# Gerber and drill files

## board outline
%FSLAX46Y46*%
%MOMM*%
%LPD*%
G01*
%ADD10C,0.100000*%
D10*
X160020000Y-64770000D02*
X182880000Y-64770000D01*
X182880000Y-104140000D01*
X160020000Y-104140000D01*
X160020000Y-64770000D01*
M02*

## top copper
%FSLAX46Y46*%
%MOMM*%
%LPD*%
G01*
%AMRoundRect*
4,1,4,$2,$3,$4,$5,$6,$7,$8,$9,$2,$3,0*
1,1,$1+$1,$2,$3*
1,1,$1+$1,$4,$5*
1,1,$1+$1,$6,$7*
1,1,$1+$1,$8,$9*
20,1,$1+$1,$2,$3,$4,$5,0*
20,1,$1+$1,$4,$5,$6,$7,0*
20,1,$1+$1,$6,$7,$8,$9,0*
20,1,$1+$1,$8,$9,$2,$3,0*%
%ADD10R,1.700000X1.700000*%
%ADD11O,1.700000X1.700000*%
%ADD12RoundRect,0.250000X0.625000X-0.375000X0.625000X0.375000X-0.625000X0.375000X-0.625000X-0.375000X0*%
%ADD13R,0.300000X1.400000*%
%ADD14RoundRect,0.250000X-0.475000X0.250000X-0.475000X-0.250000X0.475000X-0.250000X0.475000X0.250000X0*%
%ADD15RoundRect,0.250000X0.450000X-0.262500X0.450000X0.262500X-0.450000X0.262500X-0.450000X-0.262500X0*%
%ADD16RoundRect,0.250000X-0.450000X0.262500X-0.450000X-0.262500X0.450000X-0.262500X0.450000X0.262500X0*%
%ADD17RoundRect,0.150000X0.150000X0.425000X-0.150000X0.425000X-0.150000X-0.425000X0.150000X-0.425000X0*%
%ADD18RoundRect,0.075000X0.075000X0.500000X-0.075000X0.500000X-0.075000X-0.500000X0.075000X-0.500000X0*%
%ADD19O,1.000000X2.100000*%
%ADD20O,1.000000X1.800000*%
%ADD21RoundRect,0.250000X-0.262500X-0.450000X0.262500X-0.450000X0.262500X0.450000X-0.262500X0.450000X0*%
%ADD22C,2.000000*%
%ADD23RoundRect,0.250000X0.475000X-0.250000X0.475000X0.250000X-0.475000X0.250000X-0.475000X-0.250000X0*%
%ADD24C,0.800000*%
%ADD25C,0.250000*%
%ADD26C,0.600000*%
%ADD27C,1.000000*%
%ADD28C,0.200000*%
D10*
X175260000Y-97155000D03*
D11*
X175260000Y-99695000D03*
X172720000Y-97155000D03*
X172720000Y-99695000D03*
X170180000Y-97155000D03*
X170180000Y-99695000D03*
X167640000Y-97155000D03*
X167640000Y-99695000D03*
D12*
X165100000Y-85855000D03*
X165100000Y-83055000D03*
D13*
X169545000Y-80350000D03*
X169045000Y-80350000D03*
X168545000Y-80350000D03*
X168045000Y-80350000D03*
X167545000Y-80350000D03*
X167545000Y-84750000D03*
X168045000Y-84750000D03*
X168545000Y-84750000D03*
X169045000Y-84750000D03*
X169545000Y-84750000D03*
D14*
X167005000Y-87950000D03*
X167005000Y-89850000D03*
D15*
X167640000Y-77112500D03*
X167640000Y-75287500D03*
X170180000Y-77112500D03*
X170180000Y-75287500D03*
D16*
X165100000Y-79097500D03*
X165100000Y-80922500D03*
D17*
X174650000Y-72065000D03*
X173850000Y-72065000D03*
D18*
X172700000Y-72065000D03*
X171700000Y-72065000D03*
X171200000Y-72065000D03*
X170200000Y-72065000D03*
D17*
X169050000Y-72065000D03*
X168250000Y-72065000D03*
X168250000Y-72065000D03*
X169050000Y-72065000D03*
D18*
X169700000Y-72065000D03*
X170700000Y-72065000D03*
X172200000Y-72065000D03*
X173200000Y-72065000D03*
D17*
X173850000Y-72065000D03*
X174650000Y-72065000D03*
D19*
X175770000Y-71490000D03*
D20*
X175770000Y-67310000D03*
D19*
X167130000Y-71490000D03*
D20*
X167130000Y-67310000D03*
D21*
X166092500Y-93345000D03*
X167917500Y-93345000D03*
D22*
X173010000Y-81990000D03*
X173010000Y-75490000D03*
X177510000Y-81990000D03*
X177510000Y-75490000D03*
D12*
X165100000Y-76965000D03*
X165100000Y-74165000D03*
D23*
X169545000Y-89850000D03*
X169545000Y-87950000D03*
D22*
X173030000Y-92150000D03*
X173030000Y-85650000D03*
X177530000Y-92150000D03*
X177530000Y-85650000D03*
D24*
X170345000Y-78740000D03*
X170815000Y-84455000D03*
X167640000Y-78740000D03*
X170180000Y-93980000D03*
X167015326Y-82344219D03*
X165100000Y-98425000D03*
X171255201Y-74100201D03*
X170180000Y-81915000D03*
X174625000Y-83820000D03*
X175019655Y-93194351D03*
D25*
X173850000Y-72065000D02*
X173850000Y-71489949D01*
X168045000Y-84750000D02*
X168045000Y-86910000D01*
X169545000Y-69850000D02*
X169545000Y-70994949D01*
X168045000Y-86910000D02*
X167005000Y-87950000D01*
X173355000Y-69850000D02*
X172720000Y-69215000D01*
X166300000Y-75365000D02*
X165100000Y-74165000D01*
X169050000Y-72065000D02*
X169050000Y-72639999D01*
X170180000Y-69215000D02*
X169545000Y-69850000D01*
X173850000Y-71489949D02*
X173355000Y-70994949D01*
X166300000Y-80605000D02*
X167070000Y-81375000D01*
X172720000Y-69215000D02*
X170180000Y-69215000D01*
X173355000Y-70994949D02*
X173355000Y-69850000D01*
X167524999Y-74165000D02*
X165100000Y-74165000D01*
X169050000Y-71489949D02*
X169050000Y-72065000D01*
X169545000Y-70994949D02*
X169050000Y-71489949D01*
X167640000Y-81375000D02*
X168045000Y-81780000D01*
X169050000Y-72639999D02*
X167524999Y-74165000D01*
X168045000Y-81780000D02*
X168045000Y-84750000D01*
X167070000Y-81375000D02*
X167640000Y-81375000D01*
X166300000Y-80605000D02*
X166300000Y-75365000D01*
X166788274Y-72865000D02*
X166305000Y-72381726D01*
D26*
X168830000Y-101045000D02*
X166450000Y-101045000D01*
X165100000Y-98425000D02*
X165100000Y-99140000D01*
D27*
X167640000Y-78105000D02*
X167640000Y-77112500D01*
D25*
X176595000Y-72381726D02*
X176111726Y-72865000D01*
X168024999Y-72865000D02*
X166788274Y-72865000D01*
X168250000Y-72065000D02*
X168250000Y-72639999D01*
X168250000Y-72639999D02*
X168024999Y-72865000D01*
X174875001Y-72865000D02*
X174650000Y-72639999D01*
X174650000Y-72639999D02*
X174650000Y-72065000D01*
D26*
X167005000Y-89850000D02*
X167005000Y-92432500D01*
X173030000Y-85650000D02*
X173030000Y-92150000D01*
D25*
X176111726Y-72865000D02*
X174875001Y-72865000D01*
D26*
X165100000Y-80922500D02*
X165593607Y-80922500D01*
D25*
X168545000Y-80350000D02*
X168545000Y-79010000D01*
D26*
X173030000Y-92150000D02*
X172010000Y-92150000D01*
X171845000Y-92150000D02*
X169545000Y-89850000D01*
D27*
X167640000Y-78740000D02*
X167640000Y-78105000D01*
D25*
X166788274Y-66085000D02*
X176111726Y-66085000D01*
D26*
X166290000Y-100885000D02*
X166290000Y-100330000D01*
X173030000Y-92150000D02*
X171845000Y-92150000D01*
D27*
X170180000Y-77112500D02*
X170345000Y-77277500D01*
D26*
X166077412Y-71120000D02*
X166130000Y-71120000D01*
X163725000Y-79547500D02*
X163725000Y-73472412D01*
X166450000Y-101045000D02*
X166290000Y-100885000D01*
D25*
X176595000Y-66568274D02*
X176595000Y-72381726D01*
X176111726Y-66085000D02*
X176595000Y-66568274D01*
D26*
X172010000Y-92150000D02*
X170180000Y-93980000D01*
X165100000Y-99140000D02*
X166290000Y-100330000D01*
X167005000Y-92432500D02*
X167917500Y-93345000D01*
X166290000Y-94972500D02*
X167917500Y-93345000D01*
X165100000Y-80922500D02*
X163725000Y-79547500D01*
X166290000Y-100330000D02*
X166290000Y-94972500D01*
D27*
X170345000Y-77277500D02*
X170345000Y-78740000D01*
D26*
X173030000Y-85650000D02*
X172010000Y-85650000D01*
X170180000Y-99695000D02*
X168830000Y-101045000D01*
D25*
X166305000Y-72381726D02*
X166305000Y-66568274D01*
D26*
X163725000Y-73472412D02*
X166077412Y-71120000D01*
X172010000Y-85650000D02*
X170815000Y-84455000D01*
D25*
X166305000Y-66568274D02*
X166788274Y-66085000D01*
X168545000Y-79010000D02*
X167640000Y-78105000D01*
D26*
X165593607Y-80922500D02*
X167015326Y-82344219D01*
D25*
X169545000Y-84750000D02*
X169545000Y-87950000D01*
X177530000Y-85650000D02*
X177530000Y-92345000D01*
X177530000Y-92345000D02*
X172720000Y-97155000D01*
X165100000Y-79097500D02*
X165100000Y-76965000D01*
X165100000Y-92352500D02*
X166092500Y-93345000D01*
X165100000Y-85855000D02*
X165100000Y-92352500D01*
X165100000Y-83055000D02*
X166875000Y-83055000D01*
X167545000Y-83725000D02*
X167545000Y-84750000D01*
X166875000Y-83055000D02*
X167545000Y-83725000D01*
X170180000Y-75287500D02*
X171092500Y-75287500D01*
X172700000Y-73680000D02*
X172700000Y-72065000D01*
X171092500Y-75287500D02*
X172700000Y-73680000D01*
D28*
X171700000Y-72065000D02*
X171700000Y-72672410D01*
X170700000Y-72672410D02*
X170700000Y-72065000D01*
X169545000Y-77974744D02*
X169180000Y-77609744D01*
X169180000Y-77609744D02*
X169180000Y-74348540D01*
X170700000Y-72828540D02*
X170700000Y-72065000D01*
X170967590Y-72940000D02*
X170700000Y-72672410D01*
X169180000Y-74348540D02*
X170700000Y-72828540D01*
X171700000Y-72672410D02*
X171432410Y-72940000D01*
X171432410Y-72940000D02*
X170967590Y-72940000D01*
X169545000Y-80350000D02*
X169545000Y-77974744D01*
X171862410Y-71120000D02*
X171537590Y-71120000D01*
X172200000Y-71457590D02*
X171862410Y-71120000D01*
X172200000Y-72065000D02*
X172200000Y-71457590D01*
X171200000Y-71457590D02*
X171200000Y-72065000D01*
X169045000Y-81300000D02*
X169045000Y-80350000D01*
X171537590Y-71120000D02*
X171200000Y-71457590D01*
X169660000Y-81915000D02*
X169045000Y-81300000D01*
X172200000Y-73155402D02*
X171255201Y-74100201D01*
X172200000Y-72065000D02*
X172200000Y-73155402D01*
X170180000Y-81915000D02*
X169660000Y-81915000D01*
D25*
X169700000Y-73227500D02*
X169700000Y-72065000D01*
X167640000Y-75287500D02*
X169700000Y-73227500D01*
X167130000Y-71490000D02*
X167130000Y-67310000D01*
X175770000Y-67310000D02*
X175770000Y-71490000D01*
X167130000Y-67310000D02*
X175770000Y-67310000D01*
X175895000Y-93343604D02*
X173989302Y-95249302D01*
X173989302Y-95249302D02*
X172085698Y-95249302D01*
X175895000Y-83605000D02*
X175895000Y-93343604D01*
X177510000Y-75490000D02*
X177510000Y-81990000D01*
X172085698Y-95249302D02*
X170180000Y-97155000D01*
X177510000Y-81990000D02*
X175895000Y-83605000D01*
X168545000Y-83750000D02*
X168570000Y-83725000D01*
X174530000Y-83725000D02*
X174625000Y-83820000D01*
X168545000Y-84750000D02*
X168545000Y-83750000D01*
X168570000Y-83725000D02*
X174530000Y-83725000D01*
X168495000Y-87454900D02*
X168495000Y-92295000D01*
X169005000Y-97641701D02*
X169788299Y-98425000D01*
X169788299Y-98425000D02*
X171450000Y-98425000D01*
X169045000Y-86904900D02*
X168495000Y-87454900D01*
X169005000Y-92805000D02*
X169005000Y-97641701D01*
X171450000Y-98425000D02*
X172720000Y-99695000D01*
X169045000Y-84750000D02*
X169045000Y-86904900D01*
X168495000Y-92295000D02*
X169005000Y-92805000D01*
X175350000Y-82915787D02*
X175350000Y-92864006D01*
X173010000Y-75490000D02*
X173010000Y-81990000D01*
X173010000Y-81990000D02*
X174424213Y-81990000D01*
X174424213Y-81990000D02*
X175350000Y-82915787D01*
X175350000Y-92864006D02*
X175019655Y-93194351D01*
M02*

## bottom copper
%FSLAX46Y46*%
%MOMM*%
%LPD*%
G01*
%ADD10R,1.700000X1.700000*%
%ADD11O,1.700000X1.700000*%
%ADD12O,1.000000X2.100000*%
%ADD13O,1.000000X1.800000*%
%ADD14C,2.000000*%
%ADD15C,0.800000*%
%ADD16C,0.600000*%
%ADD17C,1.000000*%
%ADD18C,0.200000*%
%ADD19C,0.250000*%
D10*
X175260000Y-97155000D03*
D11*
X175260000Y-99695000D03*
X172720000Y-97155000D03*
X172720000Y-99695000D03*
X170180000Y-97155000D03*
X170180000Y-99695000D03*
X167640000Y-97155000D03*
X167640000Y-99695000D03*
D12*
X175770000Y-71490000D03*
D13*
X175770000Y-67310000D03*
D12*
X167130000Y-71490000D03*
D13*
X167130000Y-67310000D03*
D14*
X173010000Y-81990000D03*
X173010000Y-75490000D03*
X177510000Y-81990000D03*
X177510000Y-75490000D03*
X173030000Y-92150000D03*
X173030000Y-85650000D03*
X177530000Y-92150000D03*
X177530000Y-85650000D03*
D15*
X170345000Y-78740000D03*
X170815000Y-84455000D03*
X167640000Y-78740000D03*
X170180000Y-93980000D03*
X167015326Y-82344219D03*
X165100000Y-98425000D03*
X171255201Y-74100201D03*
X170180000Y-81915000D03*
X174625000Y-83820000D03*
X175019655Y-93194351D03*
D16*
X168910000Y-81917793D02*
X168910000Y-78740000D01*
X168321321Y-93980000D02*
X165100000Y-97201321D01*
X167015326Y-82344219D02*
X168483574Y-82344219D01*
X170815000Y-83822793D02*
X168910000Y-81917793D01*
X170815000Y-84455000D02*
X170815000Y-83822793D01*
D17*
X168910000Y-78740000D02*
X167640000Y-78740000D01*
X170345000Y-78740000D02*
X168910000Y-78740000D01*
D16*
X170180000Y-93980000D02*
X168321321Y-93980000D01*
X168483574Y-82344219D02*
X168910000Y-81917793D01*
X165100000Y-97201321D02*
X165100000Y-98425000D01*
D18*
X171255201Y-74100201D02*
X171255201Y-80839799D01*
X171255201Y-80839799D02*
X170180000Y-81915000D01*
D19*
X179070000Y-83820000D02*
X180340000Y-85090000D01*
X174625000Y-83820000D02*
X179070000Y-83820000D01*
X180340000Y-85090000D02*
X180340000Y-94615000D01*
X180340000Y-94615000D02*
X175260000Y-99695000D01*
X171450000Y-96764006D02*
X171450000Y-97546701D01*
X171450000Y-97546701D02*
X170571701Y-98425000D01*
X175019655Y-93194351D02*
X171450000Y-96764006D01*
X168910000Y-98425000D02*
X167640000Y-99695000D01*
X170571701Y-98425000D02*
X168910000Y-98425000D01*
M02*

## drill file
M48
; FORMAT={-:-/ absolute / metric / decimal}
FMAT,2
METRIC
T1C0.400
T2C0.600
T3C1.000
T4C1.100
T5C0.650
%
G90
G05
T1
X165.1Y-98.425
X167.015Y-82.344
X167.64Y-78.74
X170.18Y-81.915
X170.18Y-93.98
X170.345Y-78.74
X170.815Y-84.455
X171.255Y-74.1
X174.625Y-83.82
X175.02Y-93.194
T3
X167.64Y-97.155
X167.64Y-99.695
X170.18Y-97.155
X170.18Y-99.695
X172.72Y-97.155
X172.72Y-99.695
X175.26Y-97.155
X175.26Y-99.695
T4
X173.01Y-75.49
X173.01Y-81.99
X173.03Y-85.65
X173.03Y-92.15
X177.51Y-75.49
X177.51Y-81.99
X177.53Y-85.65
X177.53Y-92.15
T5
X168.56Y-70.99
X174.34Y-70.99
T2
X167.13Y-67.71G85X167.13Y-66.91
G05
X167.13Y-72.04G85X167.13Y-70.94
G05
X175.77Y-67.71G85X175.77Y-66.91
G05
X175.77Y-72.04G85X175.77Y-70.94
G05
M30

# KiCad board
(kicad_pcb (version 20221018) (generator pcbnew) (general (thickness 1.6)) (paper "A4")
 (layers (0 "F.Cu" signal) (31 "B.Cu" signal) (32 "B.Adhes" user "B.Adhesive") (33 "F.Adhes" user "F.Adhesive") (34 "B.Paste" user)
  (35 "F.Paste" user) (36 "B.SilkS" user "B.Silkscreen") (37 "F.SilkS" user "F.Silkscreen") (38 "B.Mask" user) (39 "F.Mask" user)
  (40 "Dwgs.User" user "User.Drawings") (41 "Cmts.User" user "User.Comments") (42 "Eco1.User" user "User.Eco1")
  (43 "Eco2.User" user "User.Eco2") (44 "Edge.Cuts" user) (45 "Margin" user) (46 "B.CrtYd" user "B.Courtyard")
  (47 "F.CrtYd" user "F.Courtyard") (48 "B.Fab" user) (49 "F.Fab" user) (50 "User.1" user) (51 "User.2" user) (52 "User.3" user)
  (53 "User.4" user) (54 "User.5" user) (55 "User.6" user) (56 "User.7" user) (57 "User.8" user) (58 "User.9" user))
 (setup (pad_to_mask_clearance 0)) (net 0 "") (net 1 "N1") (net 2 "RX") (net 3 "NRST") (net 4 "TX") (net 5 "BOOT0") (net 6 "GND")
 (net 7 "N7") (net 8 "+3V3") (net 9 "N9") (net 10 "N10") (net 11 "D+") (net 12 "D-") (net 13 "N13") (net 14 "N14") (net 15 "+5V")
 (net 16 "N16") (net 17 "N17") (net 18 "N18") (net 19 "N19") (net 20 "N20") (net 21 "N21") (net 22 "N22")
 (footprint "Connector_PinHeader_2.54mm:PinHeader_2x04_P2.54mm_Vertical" (layer "F.Cu") (at 175.26 97.155 -90)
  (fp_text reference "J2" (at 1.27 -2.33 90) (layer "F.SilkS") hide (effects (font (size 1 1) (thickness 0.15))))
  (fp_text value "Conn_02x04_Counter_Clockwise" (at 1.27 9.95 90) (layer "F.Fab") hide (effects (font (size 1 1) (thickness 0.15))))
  (pad "1" thru_hole rect (at 0 0 270) (size 1.7 1.7) (drill 1) (layers "*.Cu" "*.Mask") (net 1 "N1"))
  (pad "2" thru_hole oval (at 2.54 0 270) (size 1.7 1.7) (drill 1) (layers "*.Cu" "*.Mask") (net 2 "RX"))
  (pad "3" thru_hole oval (at 0 2.54 270) (size 1.7 1.7) (drill 1) (layers "*.Cu" "*.Mask") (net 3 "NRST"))
  (pad "4" thru_hole oval (at 2.54 2.54 270) (size 1.7 1.7) (drill 1) (layers "*.Cu" "*.Mask") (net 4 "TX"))
  (pad "5" thru_hole oval (at 0 5.08 270) (size 1.7 1.7) (drill 1) (layers "*.Cu" "*.Mask") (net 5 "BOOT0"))
  (pad "6" thru_hole oval (at 2.54 5.08 270) (size 1.7 1.7) (drill 1) (layers "*.Cu" "*.Mask") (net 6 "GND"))
  (pad "7" thru_hole oval (at 0 7.62 270) (size 1.7 1.7) (drill 1) (layers "*.Cu" "*.Mask") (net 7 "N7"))
  (pad "8" thru_hole oval (at 2.54 7.62 270) (size 1.7 1.7) (drill 1) (layers "*.Cu" "*.Mask") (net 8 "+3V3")))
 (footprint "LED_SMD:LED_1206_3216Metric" (layer "F.Cu") (at 165.1 84.455 90)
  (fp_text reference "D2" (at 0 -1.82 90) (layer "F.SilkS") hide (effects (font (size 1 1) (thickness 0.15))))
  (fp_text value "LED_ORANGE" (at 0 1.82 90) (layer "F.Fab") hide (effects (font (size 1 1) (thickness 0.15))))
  (pad "1" smd roundrect (at -1.4 0 90) (size 1.25 1.75) (layers "F.Cu" "F.Paste" "F.Mask") (roundrect_rratio 0.2) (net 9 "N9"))
  (pad "2" smd roundrect (at 1.4 0 90) (size 1.25 1.75) (layers "F.Cu" "F.Paste" "F.Mask") (roundrect_rratio 0.2) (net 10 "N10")))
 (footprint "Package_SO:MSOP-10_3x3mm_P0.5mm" (layer "F.Cu") (at 168.545 82.55 -90)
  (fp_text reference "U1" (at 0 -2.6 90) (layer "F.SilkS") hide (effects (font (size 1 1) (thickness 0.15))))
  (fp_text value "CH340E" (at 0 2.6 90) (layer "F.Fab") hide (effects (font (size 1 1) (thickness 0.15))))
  (pad "1" smd rect (at -2.2 -1 270) (size 1.4 0.3) (layers "F.Cu" "F.Paste" "F.Mask") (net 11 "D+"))
  (pad "2" smd rect (at -2.2 -0.5 270) (size 1.4 0.3) (layers "F.Cu" "F.Paste" "F.Mask") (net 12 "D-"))
  (pad "3" smd rect (at -2.2 0 270) (size 1.4 0.3) (layers "F.Cu" "F.Paste" "F.Mask") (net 6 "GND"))
  (pad "4" smd rect (at -2.2 0.5 270) (size 1.4 0.3) (layers "F.Cu" "F.Paste" "F.Mask") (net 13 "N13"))
  (pad "5" smd rect (at -2.2 1 270) (size 1.4 0.3) (layers "F.Cu" "F.Paste" "F.Mask") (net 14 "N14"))
  (pad "6" smd rect (at 2.2 1 270) (size 1.4 0.3) (layers "F.Cu" "F.Paste" "F.Mask") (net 10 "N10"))
  (pad "7" smd rect (at 2.2 0.5 270) (size 1.4 0.3) (layers "F.Cu" "F.Paste" "F.Mask") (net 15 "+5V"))
  (pad "8" smd rect (at 2.2 0 270) (size 1.4 0.3) (layers "F.Cu" "F.Paste" "F.Mask") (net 2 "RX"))
  (pad "9" smd rect (at 2.2 -0.5 270) (size 1.4 0.3) (layers "F.Cu" "F.Paste" "F.Mask") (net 4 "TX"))
  (pad "10" smd rect (at 2.2 -1 270) (size 1.4 0.3) (layers "F.Cu" "F.Paste" "F.Mask") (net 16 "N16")))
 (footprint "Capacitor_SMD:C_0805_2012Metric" (layer "F.Cu") (at 167.005 88.9 -90)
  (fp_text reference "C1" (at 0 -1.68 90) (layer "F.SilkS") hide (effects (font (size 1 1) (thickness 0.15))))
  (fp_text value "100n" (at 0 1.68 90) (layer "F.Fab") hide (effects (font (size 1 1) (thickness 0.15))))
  (pad "1" smd roundrect (at -0.95 0 270) (size 1 1.45) (layers "F.Cu" "F.Paste" "F.Mask") (roundrect_rratio 0.25) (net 15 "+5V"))
  (pad "2" smd roundrect (at 0.95 0 270) (size 1 1.45) (layers "F.Cu" "F.Paste" "F.Mask") (roundrect_rratio 0.25) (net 6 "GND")))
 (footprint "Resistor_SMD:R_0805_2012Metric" (layer "F.Cu") (at 167.64 76.2 90)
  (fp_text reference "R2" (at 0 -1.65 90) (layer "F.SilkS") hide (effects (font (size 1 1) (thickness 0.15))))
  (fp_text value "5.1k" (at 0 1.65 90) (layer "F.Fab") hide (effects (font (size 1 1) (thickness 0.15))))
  (pad "1" smd roundrect (at -0.9125 0 90) (size 1.025 1.4) (layers "F.Cu" "F.Paste" "F.Mask") (roundrect_rratio 0.243902439) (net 6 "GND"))
  (pad "2" smd roundrect (at 0.9125 0 90) (size 1.025 1.4) (layers "F.Cu" "F.Paste" "F.Mask") (roundrect_rratio 0.243902439) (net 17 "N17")))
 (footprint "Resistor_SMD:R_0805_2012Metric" (layer "F.Cu") (at 170.18 76.2 90)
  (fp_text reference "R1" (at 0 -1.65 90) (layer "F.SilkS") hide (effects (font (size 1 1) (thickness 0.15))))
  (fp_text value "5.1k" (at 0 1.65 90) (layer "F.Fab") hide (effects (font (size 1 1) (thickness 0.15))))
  (pad "1" smd roundrect (at -0.9125 0 90) (size 1.025 1.4) (layers "F.Cu" "F.Paste" "F.Mask") (roundrect_rratio 0.243902439) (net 6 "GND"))
  (pad "2" smd roundrect (at 0.9125 0 90) (size 1.025 1.4) (layers "F.Cu" "F.Paste" "F.Mask") (roundrect_rratio 0.243902439) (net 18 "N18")))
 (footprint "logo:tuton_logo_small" (layer "F.Cu") (at 162.56 69.215 90)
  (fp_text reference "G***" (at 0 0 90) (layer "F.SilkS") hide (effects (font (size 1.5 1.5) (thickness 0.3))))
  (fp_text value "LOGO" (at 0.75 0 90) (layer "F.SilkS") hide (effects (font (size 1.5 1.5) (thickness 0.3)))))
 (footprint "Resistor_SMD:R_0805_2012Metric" (layer "F.Cu") (at 165.1 80.01 -90)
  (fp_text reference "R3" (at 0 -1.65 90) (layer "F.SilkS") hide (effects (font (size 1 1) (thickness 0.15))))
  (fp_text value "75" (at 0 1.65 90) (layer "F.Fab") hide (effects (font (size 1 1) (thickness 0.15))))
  (pad "1" smd roundrect (at -0.9125 0 270) (size 1.025 1.4) (layers "F.Cu" "F.Paste" "F.Mask") (roundrect_rratio 0.243902439)
   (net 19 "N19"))
  (pad "2" smd roundrect (at 0.9125 0 270) (size 1.025 1.4) (layers "F.Cu" "F.Paste" "F.Mask") (roundrect_rratio 0.243902439) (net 6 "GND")))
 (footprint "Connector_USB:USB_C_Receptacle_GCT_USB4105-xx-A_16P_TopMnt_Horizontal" (layer "F.Cu") (at 171.45 68.385 180)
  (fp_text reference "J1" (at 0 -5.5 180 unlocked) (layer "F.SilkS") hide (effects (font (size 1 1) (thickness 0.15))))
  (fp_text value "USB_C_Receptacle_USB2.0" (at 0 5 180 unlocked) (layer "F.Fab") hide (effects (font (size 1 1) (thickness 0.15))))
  (pad "" np_thru_hole circle (at -2.89 -2.605 180) (size 0.65 0.65) (drill 0.65) (layers "F&B.Cu" "*.Mask"))
  (pad "" np_thru_hole circle (at 2.89 -2.605 180) (size 0.65 0.65) (drill 0.65) (layers "F&B.Cu" "*.Mask"))
  (pad "A1" smd roundrect (at -3.2 -3.68 180) (size 0.6 1.15) (layers "F.Cu" "F.Paste" "F.Mask") (roundrect_rratio 0.25) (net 6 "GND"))
  (pad "A4" smd roundrect (at -2.4 -3.68 180) (size 0.6 1.15) (layers "F.Cu" "F.Paste" "F.Mask") (roundrect_rratio 0.25) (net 15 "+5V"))
  (pad "A5" smd roundrect (at -1.25 -3.68 180) (size 0.3 1.15) (layers "F.Cu" "F.Paste" "F.Mask") (roundrect_rratio 0.25) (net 18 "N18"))
  (pad "A6" smd roundrect (at -0.25 -3.68 180) (size 0.3 1.15) (layers "F.Cu" "F.Paste" "F.Mask") (roundrect_rratio 0.25) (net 11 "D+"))
  (pad "A7" smd roundrect (at 0.25 -3.68 180) (size 0.3 1.15) (layers "F.Cu" "F.Paste" "F.Mask") (roundrect_rratio 0.25) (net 12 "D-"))
  (pad "A8" smd roundrect (at 1.25 -3.68 180) (size 0.3 1.15) (layers "F.Cu" "F.Paste" "F.Mask") (roundrect_rratio 0.25) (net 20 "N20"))
  (pad "A9" smd roundrect (at 2.4 -3.68 180) (size 0.6 1.15) (layers "F.Cu" "F.Paste" "F.Mask") (roundrect_rratio 0.25) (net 15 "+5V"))
  (pad "A12" smd roundrect (at 3.2 -3.68 180) (size 0.6 1.15) (layers "F.Cu" "F.Paste" "F.Mask") (roundrect_rratio 0.25) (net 6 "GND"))
  (pad "B1" smd roundrect (at 3.2 -3.68 180) (size 0.6 1.15) (layers "F.Cu" "F.Paste" "F.Mask") (roundrect_rratio 0.25) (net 6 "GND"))
  (pad "B4" smd roundrect (at 2.4 -3.68 180) (size 0.6 1.15) (layers "F.Cu" "F.Paste" "F.Mask") (roundrect_rratio 0.25) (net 15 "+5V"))
  (pad "B5" smd roundrect (at 1.75 -3.68 180) (size 0.3 1.15) (layers "F.Cu" "F.Paste" "F.Mask") (roundrect_rratio 0.25) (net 17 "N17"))
  (pad "B6" smd roundrect (at 0.75 -3.68 180) (size 0.3 1.15) (layers "F.Cu" "F.Paste" "F.Mask") (roundrect_rratio 0.25) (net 11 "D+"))
  (pad "B7" smd roundrect (at -0.75 -3.68 180) (size 0.3 1.15) (layers "F.Cu" "F.Paste" "F.Mask") (roundrect_rratio 0.25) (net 12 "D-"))
  (pad "B8" smd roundrect (at -1.75 -3.68 180) (size 0.3 1.15) (layers "F.Cu" "F.Paste" "F.Mask") (roundrect_rratio 0.25) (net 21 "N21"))
  (pad "B9" smd roundrect (at -2.4 -3.68 180) (size 0.6 1.15) (layers "F.Cu" "F.Paste" "F.Mask") (roundrect_rratio 0.25) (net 15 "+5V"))
  (pad "B12" smd roundrect (at -3.2 -3.68 180) (size 0.6 1.15) (layers "F.Cu" "F.Paste" "F.Mask") (roundrect_rratio 0.25) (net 6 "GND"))
  (pad "S1" thru_hole oval (at -4.32 -3.105 180) (size 1 2.1) (drill oval 0.6 1.7) (layers "*.Cu" "*.Mask" "F.Paste") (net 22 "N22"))
  (pad "S1" thru_hole oval (at -4.32 1.075 180) (size 1 1.8) (drill oval 0.6 1.4) (layers "*.Cu" "*.Mask" "F.Paste") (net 22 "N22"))
  (pad "S1" thru_hole oval (at 4.32 -3.105 180) (size 1 2.1) (drill oval 0.6 1.7) (layers "*.Cu" "*.Mask" "F.Paste") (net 22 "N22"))
  (pad "S1" thru_hole oval (at 4.32 1.075 180) (size 1 1.8) (drill oval 0.6 1.4) (layers "*.Cu" "*.Mask" "F.Paste") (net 22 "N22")))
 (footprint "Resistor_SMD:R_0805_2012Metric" (layer "F.Cu") (at 167.005 93.345)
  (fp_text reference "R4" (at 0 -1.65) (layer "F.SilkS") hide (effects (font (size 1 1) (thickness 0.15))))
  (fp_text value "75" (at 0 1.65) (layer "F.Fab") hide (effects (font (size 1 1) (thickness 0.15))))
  (pad "1" smd roundrect (at -0.9125 0) (size 1.025 1.4) (layers "F.Cu" "F.Paste" "F.Mask") (roundrect_rratio 0.243902439) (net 9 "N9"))
  (pad "2" smd roundrect (at 0.9125 0) (size 1.025 1.4) (layers "F.Cu" "F.Paste" "F.Mask") (roundrect_rratio 0.243902439) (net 6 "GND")))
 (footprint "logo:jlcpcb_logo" (layer "F.Cu") (at 162.56 86.995 90)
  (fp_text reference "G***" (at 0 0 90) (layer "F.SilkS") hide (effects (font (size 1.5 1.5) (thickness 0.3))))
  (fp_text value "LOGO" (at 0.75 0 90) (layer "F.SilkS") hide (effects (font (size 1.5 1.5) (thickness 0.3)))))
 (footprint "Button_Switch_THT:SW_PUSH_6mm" (layer "F.Cu") (at 173.01 81.99 90)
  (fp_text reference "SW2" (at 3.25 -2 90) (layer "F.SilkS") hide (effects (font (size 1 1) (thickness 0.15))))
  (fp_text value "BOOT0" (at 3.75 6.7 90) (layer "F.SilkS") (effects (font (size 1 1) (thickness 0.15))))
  (pad "1" thru_hole circle (at 0 0 180) (size 2 2) (drill 1.1) (layers "*.Cu" "*.Mask") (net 8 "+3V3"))
  (pad "1" thru_hole circle (at 6.5 0 180) (size 2 2) (drill 1.1) (layers "*.Cu" "*.Mask") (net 8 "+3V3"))
  (pad "2" thru_hole circle (at 0 4.5 180) (size 2 2) (drill 1.1) (layers "*.Cu" "*.Mask") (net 5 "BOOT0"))
  (pad "2" thru_hole circle (at 6.5 4.5 180) (size 2 2) (drill 1.1) (layers "*.Cu" "*.Mask") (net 5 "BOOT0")))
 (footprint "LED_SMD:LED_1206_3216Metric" (layer "F.Cu") (at 165.1 75.565 90)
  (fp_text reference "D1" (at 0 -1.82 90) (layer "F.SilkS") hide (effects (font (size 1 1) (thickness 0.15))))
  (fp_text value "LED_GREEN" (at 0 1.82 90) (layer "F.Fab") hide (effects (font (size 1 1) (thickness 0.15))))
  (pad "1" smd roundrect (at -1.4 0 90) (size 1.25 1.75) (layers "F.Cu" "F.Paste" "F.Mask") (roundrect_rratio 0.2) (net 19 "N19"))
  (pad "2" smd roundrect (at 1.4 0 90) (size 1.25 1.75) (layers "F.Cu" "F.Paste" "F.Mask") (roundrect_rratio 0.2) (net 15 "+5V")))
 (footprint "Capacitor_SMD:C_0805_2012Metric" (layer "F.Cu") (at 169.545 88.9 90)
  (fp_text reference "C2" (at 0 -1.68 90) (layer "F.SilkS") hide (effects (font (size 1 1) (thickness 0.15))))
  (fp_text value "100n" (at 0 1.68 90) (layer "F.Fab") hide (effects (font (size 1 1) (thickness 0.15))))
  (pad "1" smd roundrect (at -0.95 0 90) (size 1 1.45) (layers "F.Cu" "F.Paste" "F.Mask") (roundrect_rratio 0.25) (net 6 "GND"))
  (pad "2" smd roundrect (at 0.95 0 90) (size 1 1.45) (layers "F.Cu" "F.Paste" "F.Mask") (roundrect_rratio 0.25) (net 16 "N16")))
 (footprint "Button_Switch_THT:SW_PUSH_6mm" (layer "F.Cu") (at 173.03 92.15 90)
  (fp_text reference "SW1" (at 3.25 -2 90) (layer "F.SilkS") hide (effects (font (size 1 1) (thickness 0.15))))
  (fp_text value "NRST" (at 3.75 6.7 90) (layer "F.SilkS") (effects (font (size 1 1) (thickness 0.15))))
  (pad "1" thru_hole circle (at 0 0 180) (size 2 2) (drill 1.1) (layers "*.Cu" "*.Mask") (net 6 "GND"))
  (pad "1" thru_hole circle (at 6.5 0 180) (size 2 2) (drill 1.1) (layers "*.Cu" "*.Mask") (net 6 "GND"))
  (pad "2" thru_hole circle (at 0 4.5 180) (size 2 2) (drill 1.1) (layers "*.Cu" "*.Mask") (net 3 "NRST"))
  (pad "2" thru_hole circle (at 6.5 4.5 180) (size 2 2) (drill 1.1) (layers "*.Cu" "*.Mask") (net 3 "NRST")))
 (gr_rect (start 160.02 64.77) (end 182.88 104.14) (stroke (width 0.1) (type default)) (fill none) (layer "Edge.Cuts"))
 (segment (start 173.85 72.065) (end 173.85 71.489949) (width 0.25) (layer "F.Cu") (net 15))
 (segment (start 168.045 84.75) (end 168.045 86.91) (width 0.25) (layer "F.Cu") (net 15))
 (segment (start 169.545 69.85) (end 169.545 70.994949) (width 0.25) (layer "F.Cu") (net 15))
 (segment (start 168.045 86.91) (end 167.005 87.95) (width 0.25) (layer "F.Cu") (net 15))
 (segment (start 173.355 69.85) (end 172.72 69.215) (width 0.25) (layer "F.Cu") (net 15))
 (segment (start 166.3 75.365) (end 165.1 74.165) (width 0.25) (layer "F.Cu") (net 15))
 (segment (start 169.05 72.065) (end 169.05 72.639999) (width 0.25) (layer "F.Cu") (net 15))
 (segment (start 170.18 69.215) (end 169.545 69.85) (width 0.25) (layer "F.Cu") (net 15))
 (segment (start 173.85 71.489949) (end 173.355 70.994949) (width 0.25) (layer "F.Cu") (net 15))
 (segment (start 166.3 80.605) (end 167.07 81.375) (width 0.25) (layer "F.Cu") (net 15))
 (segment (start 172.72 69.215) (end 170.18 69.215) (width 0.25) (layer "F.Cu") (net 15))
 (segment (start 173.355 70.994949) (end 173.355 69.85) (width 0.25) (layer "F.Cu") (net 15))
 (segment (start 167.524999 74.165) (end 165.1 74.165) (width 0.25) (layer "F.Cu") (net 15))
 (segment (start 169.05 71.489949) (end 169.05 72.065) (width 0.25) (layer "F.Cu") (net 15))
 (segment (start 169.545 70.994949) (end 169.05 71.489949) (width 0.25) (layer "F.Cu") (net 15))
 (segment (start 167.64 81.375) (end 168.045 81.78) (width 0.25) (layer "F.Cu") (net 15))
 (segment (start 169.05 72.639999) (end 167.524999 74.165) (width 0.25) (layer "F.Cu") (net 15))
 (segment (start 168.045 81.78) (end 168.045 84.75) (width 0.25) (layer "F.Cu") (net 15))
 (segment (start 167.07 81.375) (end 167.64 81.375) (width 0.25) (layer "F.Cu") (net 15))
 (segment (start 166.3 80.605) (end 166.3 75.365) (width 0.25) (layer "F.Cu") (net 15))
 (segment (start 166.788274 72.865) (end 166.305 72.381726) (width 0.25) (layer "F.Cu") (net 6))
 (segment (start 168.83 101.045) (end 166.45 101.045) (width 0.6) (layer "F.Cu") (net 6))
 (segment (start 165.1 98.425) (end 165.1 99.14) (width 0.6) (layer "F.Cu") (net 6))
 (segment (start 167.64 78.105) (end 167.64 77.1125) (width 1) (layer "F.Cu") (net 6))
 (segment (start 176.595 72.381726) (end 176.111726 72.865) (width 0.25) (layer "F.Cu") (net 6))
 (segment (start 168.024999 72.865) (end 166.788274 72.865) (width 0.25) (layer "F.Cu") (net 6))
 (segment (start 168.25 72.065) (end 168.25 72.639999) (width 0.25) (layer "F.Cu") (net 6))
 (segment (start 168.25 72.639999) (end 168.024999 72.865) (width 0.25) (layer "F.Cu") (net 6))
 (segment (start 174.875001 72.865) (end 174.65 72.639999) (width 0.25) (layer "F.Cu") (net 6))
 (segment (start 174.65 72.639999) (end 174.65 72.065) (width 0.25) (layer "F.Cu") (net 6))
 (segment (start 167.005 89.85) (end 167.005 92.4325) (width 0.6) (layer "F.Cu") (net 6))
 (segment (start 173.03 85.65) (end 173.03 92.15) (width 0.6) (layer "F.Cu") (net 6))
 (segment (start 176.111726 72.865) (end 174.875001 72.865) (width 0.25) (layer "F.Cu") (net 6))
 (segment (start 165.1 80.9225) (end 165.593607 80.9225) (width 0.6) (layer "F.Cu") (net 6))
 (segment (start 168.545 80.35) (end 168.545 79.01) (width 0.25) (layer "F.Cu") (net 6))
 (segment (start 173.03 92.15) (end 172.01 92.15) (width 0.6) (layer "F.Cu") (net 6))
 (segment (start 171.845 92.15) (end 169.545 89.85) (width 0.6) (layer "F.Cu") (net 6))
 (segment (start 167.64 78.74) (end 167.64 78.105) (width 1) (layer "F.Cu") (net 6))
 (segment (start 166.788274 66.085) (end 176.111726 66.085) (width 0.25) (layer "F.Cu") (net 6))
 (segment (start 166.29 100.885) (end 166.29 100.33) (width 0.6) (layer "F.Cu") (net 6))
 (segment (start 173.03 92.15) (end 171.845 92.15) (width 0.6) (layer "F.Cu") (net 6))
 (segment (start 170.18 77.1125) (end 170.345 77.2775) (width 1) (layer "F.Cu") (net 6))
 (segment (start 166.077412 71.12) (end 166.13 71.12) (width 0.6) (layer "F.Cu") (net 6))
 (segment (start 163.725 79.5475) (end 163.725 73.472412) (width 0.6) (layer "F.Cu") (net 6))
 (segment (start 166.45 101.045) (end 166.29 100.885) (width 0.6) (layer "F.Cu") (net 6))
 (segment (start 176.595 66.568274) (end 176.595 72.381726) (width 0.25) (layer "F.Cu") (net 6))
 (segment (start 176.111726 66.085) (end 176.595 66.568274) (width 0.25) (layer "F.Cu") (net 6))
 (segment (start 172.01 92.15) (end 170.18 93.98) (width 0.6) (layer "F.Cu") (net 6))
 (segment (start 165.1 99.14) (end 166.29 100.33) (width 0.6) (layer "F.Cu") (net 6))
 (segment (start 167.005 92.4325) (end 167.9175 93.345) (width 0.6) (layer "F.Cu") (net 6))
 (segment (start 166.29 94.9725) (end 167.9175 93.345) (width 0.6) (layer "F.Cu") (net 6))
 (segment (start 165.1 80.9225) (end 163.725 79.5475) (width 0.6) (layer "F.Cu") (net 6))
 (segment (start 166.29 100.33) (end 166.29 94.9725) (width 0.6) (layer "F.Cu") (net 6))
 (segment (start 170.345 77.2775) (end 170.345 78.74) (width 1) (layer "F.Cu") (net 6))
 (segment (start 173.03 85.65) (end 172.01 85.65) (width 0.6) (layer "F.Cu") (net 6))
 (segment (start 170.18 99.695) (end 168.83 101.045) (width 0.6) (layer "F.Cu") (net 6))
 (segment (start 166.305 72.381726) (end 166.305 66.568274) (width 0.25) (layer "F.Cu") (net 6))
 (segment (start 163.725 73.472412) (end 166.077412 71.12) (width 0.6) (layer "F.Cu") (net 6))
 (segment (start 172.01 85.65) (end 170.815 84.455) (width 0.6) (layer "F.Cu") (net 6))
 (segment (start 166.305 66.568274) (end 166.788274 66.085) (width 0.25) (layer "F.Cu") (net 6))
 (segment (start 168.545 79.01) (end 167.64 78.105) (width 0.25) (layer "F.Cu") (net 6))
 (segment (start 165.593607 80.9225) (end 167.015326 82.344219) (width 0.6) (layer "F.Cu") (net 6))
 (via (at 170.345 78.74) (size 0.8) (drill 0.4) (layers "F.Cu" "B.Cu") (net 6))
 (via (at 170.815 84.455) (size 0.8) (drill 0.4) (layers "F.Cu" "B.Cu") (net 6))
 (via (at 167.64 78.74) (size 0.8) (drill 0.4) (layers "F.Cu" "B.Cu") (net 6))
 (via (at 170.18 93.98) (size 0.8) (drill 0.4) (layers "F.Cu" "B.Cu") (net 6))
 (via (at 167.015326 82.344219) (size 0.8) (drill 0.4) (layers "F.Cu" "B.Cu") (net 6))
 (via (at 165.1 98.425) (size 0.8) (drill 0.4) (layers "F.Cu" "B.Cu") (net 6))
 (segment (start 168.91 81.917793) (end 168.91 78.74) (width 0.6) (layer "B.Cu") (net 6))
 (segment (start 168.321321 93.98) (end 165.1 97.201321) (width 0.6) (layer "B.Cu") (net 6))
 (segment (start 167.015326 82.344219) (end 168.483574 82.344219) (width 0.6) (layer "B.Cu") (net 6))
 (segment (start 170.815 83.822793) (end 168.91 81.917793) (width 0.6) (layer "B.Cu") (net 6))
 (segment (start 170.815 84.455) (end 170.815 83.822793) (width 0.6) (layer "B.Cu") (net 6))
 (segment (start 168.91 78.74) (end 167.64 78.74) (width 1) (layer "B.Cu") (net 6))
 (segment (start 170.345 78.74) (end 168.91 78.74) (width 1) (layer "B.Cu") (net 6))
 (segment (start 170.18 93.98) (end 168.321321 93.98) (width 0.6) (layer "B.Cu") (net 6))
 (segment (start 168.483574 82.344219) (end 168.91 81.917793) (width 0.6) (layer "B.Cu") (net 6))
 (segment (start 165.1 97.201321) (end 165.1 98.425) (width 0.6) (layer "B.Cu") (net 6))
 (segment (start 169.545 84.75) (end 169.545 87.95) (width 0.25) (layer "F.Cu") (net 16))
 (segment (start 177.53 85.65) (end 177.53 92.345) (width 0.25) (layer "F.Cu") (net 3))
 (segment (start 177.53 92.345) (end 172.72 97.155) (width 0.25) (layer "F.Cu") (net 3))
 (segment (start 165.1 79.0975) (end 165.1 76.965) (width 0.25) (layer "F.Cu") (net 19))
 (segment (start 165.1 92.3525) (end 166.0925 93.345) (width 0.25) (layer "F.Cu") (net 9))
 (segment (start 165.1 85.855) (end 165.1 92.3525) (width 0.25) (layer "F.Cu") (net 9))
 (segment (start 165.1 83.055) (end 166.875 83.055) (width 0.25) (layer "F.Cu") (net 10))
 (segment (start 167.545 83.725) (end 167.545 84.75) (width 0.25) (layer "F.Cu") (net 10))
 (segment (start 166.875 83.055) (end 167.545 83.725) (width 0.25) (layer "F.Cu") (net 10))
 (segment (start 170.18 75.2875) (end 171.0925 75.2875) (width 0.25) (layer "F.Cu") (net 18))
 (segment (start 172.7 73.68) (end 172.7 72.065) (width 0.25) (layer "F.Cu") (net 18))
 (segment (start 171.0925 75.2875) (end 172.7 73.68) (width 0.25) (layer "F.Cu") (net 18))
 (segment (start 171.7 72.065) (end 171.7 72.67241) (width 0.2) (layer "F.Cu") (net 11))
 (segment (start 170.7 72.67241) (end 170.7 72.065) (width 0.2) (layer "F.Cu") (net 11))
 (segment (start 169.545 77.974744) (end 169.18 77.609744) (width 0.2) (layer "F.Cu") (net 11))
 (segment (start 169.18 77.609744) (end 169.18 74.34854) (width 0.2) (layer "F.Cu") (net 11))
 (segment (start 170.7 72.82854) (end 170.7 72.065) (width 0.2) (layer "F.Cu") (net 11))
 (segment (start 170.96759 72.94) (end 170.7 72.67241) (width 0.2) (layer "F.Cu") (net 11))
 (segment (start 169.18 74.34854) (end 170.7 72.82854) (width 0.2) (layer "F.Cu") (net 11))
 (segment (start 171.7 72.67241) (end 171.43241 72.94) (width 0.2) (layer "F.Cu") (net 11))
 (segment (start 171.43241 72.94) (end 170.96759 72.94) (width 0.2) (layer "F.Cu") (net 11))
 (segment (start 169.545 80.35) (end 169.545 77.974744) (width 0.2) (layer "F.Cu") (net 11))
 (segment (start 171.86241 71.12) (end 171.53759 71.12) (width 0.2) (layer "F.Cu") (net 12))
 (segment (start 172.2 71.45759) (end 171.86241 71.12) (width 0.2) (layer "F.Cu") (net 12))
 (segment (start 172.2 72.065) (end 172.2 71.45759) (width 0.2) (layer "F.Cu") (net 12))
 (segment (start 171.2 71.45759) (end 171.2 72.065) (width 0.2) (layer "F.Cu") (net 12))
 (segment (start 169.045 81.3) (end 169.045 80.35) (width 0.2) (layer "F.Cu") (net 12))
 (segment (start 171.53759 71.12) (end 171.2 71.45759) (width 0.2) (layer "F.Cu") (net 12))
 (segment (start 169.66 81.915) (end 169.045 81.3) (width 0.2) (layer "F.Cu") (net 12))
 (segment (start 172.2 73.155402) (end 171.255201 74.100201) (width 0.2) (layer "F.Cu") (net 12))
 (segment (start 172.2 72.065) (end 172.2 73.155402) (width 0.2) (layer "F.Cu") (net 12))
 (segment (start 170.18 81.915) (end 169.66 81.915) (width 0.2) (layer "F.Cu") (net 12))
 (via (at 171.255201 74.100201) (size 0.8) (drill 0.4) (layers "F.Cu" "B.Cu") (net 12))
 (via (at 170.18 81.915) (size 0.8) (drill 0.4) (layers "F.Cu" "B.Cu") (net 12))
 (segment (start 171.255201 74.100201) (end 171.255201 80.839799) (width 0.2) (layer "B.Cu") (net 12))
 (segment (start 171.255201 80.839799) (end 170.18 81.915) (width 0.2) (layer "B.Cu") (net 12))
 (segment (start 169.7 73.2275) (end 169.7 72.065) (width 0.25) (layer "F.Cu") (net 17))
 (segment (start 167.64 75.2875) (end 169.7 73.2275) (width 0.25) (layer "F.Cu") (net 17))
 (segment (start 167.13 71.49) (end 167.13 67.31) (width 0.25) (layer "F.Cu") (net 22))
 (segment (start 175.77 67.31) (end 175.77 71.49) (width 0.25) (layer "F.Cu") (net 22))
 (segment (start 167.13 67.31) (end 175.77 67.31) (width 0.25) (layer "F.Cu") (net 22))
 (segment (start 175.895 93.343604) (end 173.989302 95.249302) (width 0.25) (layer "F.Cu") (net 5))
 (segment (start 173.989302 95.249302) (end 172.085698 95.249302) (width 0.25) (layer "F.Cu") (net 5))
 (segment (start 175.895 83.605) (end 175.895 93.343604) (width 0.25) (layer "F.Cu") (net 5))
 (segment (start 177.51 75.49) (end 177.51 81.99) (width 0.25) (layer "F.Cu") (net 5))
 (segment (start 172.085698 95.249302) (end 170.18 97.155) (width 0.25) (layer "F.Cu") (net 5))
 (segment (start 177.51 81.99) (end 175.895 83.605) (width 0.25) (layer "F.Cu") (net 5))
 (segment (start 168.545 83.75) (end 168.57 83.725) (width 0.25) (layer "F.Cu") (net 2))
 (segment (start 174.53 83.725) (end 174.625 83.82) (width 0.25) (layer "F.Cu") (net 2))
 (segment (start 168.545 84.75) (end 168.545 83.75) (width 0.25) (layer "F.Cu") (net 2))
 (segment (start 168.57 83.725) (end 174.53 83.725) (width 0.25) (layer "F.Cu") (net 2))
 (via (at 174.625 83.82) (size 0.8) (drill 0.4) (layers "F.Cu" "B.Cu") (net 2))
 (segment (start 179.07 83.82) (end 180.34 85.09) (width 0.25) (layer "B.Cu") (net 2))
 (segment (start 174.625 83.82) (end 179.07 83.82) (width 0.25) (layer "B.Cu") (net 2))
 (segment (start 180.34 85.09) (end 180.34 94.615) (width 0.25) (layer "B.Cu") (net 2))
 (segment (start 180.34 94.615) (end 175.26 99.695) (width 0.25) (layer "B.Cu") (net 2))
 (segment (start 168.495 87.4549) (end 168.495 92.295) (width 0.25) (layer "F.Cu") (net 4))
 (segment (start 169.005 97.641701) (end 169.788299 98.425) (width 0.25) (layer "F.Cu") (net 4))
 (segment (start 169.788299 98.425) (end 171.45 98.425) (width 0.25) (layer "F.Cu") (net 4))
 (segment (start 169.045 86.9049) (end 168.495 87.4549) (width 0.25) (layer "F.Cu") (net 4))
 (segment (start 169.005 92.805) (end 169.005 97.641701) (width 0.25) (layer "F.Cu") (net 4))
 (segment (start 171.45 98.425) (end 172.72 99.695) (width 0.25) (layer "F.Cu") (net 4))
 (segment (start 169.045 84.75) (end 169.045 86.9049) (width 0.25) (layer "F.Cu") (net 4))
 (segment (start 168.495 92.295) (end 169.005 92.805) (width 0.25) (layer "F.Cu") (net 4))
 (segment (start 175.35 82.915787) (end 175.35 92.864006) (width 0.25) (layer "F.Cu") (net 8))
 (segment (start 173.01 75.49) (end 173.01 81.99) (width 0.25) (layer "F.Cu") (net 8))
 (segment (start 173.01 81.99) (end 174.424213 81.99) (width 0.25) (layer "F.Cu") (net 8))
 (segment (start 174.424213 81.99) (end 175.35 82.915787) (width 0.25) (layer "F.Cu") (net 8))
 (segment (start 175.35 92.864006) (end 175.019655 93.194351) (width 0.25) (layer "F.Cu") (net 8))
 (via (at 175.019655 93.194351) (size 0.8) (drill 0.4) (layers "F.Cu" "B.Cu") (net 8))
 (segment (start 171.45 96.764006) (end 171.45 97.546701) (width 0.25) (layer "B.Cu") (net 8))
 (segment (start 171.45 97.546701) (end 170.571701 98.425) (width 0.25) (layer "B.Cu") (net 8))
 (segment (start 175.019655 93.194351) (end 171.45 96.764006) (width 0.25) (layer "B.Cu") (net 8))
 (segment (start 168.91 98.425) (end 167.64 99.695) (width 0.25) (layer "B.Cu") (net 8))
 (segment (start 170.571701 98.425) (end 168.91 98.425) (width 0.25) (layer "B.Cu") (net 8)))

